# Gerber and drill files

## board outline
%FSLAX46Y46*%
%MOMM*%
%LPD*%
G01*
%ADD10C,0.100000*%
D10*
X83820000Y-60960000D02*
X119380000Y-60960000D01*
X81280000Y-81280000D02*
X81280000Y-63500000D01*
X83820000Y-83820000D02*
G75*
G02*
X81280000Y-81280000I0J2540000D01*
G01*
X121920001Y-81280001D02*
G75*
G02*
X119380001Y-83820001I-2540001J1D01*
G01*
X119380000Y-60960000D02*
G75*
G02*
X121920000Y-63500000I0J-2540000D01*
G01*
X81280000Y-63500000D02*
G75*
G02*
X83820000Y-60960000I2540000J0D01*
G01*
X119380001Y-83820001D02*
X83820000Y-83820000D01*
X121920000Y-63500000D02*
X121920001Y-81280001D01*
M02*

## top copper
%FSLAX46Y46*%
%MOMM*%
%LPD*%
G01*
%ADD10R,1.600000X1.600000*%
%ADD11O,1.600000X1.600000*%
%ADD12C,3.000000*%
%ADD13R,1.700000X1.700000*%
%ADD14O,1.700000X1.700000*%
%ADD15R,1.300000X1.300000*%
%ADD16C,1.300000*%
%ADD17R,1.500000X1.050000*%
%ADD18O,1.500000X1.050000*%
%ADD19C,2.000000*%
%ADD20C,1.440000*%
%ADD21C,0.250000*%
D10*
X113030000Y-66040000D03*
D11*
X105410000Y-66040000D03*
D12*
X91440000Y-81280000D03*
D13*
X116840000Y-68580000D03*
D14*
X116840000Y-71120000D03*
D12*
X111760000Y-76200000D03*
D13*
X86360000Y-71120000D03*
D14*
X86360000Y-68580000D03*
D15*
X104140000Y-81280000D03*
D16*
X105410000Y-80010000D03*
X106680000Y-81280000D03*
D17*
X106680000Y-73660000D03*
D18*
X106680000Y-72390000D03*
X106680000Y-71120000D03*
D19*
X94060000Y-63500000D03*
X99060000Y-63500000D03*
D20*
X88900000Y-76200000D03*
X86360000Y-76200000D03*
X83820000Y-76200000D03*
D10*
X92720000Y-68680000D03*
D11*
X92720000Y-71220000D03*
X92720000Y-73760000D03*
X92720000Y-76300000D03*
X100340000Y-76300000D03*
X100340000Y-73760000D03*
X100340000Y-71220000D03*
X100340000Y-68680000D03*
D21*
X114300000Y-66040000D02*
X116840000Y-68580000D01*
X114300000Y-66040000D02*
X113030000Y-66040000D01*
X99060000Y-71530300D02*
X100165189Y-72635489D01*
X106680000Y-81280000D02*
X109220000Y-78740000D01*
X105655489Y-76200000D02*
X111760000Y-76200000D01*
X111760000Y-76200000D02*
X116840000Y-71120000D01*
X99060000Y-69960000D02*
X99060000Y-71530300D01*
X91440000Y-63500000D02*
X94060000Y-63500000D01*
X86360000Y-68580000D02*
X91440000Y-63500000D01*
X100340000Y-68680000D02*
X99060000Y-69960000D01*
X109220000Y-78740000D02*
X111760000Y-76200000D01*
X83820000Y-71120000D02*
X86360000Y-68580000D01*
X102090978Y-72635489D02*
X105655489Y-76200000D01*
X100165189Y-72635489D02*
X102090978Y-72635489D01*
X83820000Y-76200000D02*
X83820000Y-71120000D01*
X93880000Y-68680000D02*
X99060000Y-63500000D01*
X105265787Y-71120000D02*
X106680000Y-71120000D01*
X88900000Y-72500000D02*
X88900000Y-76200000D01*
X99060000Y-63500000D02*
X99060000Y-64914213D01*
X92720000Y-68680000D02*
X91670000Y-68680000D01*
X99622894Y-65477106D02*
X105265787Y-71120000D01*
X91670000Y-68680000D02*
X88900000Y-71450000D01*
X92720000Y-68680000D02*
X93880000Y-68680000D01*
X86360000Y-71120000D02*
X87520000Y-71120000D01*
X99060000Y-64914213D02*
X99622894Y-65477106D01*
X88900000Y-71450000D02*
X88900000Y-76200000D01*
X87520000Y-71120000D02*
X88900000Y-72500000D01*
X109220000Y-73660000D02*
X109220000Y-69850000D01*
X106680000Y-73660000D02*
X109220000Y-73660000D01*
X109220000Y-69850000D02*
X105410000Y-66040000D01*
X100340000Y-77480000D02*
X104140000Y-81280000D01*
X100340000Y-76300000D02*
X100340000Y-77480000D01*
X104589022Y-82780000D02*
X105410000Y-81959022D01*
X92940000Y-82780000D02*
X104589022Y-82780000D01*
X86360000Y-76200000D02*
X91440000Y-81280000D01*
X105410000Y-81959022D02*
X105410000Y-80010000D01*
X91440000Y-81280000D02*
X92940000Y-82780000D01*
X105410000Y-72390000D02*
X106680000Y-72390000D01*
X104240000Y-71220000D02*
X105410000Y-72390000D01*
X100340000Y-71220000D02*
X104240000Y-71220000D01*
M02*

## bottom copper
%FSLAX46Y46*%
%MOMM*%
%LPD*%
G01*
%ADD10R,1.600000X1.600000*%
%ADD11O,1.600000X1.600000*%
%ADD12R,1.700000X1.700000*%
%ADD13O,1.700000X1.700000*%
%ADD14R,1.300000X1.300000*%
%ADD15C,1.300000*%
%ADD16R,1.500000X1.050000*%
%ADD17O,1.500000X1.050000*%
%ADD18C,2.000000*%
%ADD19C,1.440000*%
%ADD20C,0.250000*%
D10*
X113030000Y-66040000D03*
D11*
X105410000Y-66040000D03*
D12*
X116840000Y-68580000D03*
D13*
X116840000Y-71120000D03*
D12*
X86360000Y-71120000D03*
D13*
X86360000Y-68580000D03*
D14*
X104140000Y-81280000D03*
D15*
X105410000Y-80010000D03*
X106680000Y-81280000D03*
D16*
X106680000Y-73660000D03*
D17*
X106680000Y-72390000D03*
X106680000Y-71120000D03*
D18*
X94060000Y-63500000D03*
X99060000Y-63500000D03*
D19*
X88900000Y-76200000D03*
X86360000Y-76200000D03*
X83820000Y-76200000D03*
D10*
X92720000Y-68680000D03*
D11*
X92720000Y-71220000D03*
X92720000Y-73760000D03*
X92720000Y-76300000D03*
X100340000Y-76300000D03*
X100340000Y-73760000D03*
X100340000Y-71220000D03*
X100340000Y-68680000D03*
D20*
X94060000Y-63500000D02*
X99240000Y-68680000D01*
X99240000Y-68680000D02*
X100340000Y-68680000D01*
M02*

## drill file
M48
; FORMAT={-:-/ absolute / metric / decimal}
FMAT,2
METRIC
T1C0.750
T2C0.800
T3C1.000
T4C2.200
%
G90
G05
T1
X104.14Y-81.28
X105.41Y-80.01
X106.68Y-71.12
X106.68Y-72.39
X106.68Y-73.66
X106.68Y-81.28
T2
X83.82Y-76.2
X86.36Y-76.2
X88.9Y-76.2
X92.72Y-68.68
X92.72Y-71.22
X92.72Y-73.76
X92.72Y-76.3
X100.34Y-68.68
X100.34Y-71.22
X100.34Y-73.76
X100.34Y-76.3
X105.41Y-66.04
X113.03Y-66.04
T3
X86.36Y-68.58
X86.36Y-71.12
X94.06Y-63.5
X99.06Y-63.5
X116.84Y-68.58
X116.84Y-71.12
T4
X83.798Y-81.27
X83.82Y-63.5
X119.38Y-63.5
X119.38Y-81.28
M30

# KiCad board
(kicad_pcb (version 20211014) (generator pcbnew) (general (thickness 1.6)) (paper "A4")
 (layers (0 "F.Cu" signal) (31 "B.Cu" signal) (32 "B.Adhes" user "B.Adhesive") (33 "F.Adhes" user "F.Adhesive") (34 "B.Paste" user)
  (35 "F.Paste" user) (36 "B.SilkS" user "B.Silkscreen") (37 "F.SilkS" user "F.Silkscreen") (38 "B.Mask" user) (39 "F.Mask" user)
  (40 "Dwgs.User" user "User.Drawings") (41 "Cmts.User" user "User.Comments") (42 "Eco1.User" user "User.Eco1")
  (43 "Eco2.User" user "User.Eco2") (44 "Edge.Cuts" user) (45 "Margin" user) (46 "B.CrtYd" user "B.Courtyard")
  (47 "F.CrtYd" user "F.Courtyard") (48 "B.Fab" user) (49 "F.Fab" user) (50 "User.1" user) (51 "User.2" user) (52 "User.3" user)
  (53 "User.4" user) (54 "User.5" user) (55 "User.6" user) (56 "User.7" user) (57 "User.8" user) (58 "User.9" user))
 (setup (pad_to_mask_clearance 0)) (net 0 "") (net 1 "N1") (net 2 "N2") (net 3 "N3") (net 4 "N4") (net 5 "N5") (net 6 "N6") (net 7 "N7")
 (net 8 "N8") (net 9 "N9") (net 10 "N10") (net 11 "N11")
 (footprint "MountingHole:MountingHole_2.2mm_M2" (layer "F.Cu") (at 83.82 63.5)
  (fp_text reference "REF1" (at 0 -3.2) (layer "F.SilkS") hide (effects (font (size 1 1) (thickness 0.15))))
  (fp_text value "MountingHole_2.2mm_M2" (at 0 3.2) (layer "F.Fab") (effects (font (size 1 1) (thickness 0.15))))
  (pad "" np_thru_hole circle (at 0 0) (size 2.2 2.2) (drill 2.2) (layers *.Cu *.Mask)))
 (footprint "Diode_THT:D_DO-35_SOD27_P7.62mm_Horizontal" (layer "F.Cu") (at 113.03 66.04 180)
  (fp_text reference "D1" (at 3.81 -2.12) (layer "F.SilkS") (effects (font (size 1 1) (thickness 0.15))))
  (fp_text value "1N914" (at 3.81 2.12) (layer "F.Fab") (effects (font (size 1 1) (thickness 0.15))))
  (pad "1" thru_hole rect (at 0 0 180) (size 1.6 1.6) (drill 0.8) (layers *.Cu *.Mask) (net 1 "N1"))
  (pad "2" thru_hole oval (at 7.62 0 180) (size 1.6 1.6) (drill 0.8) (layers *.Cu *.Mask) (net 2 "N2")))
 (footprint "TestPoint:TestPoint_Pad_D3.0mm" (layer "F.Cu") (at 91.44 81.28)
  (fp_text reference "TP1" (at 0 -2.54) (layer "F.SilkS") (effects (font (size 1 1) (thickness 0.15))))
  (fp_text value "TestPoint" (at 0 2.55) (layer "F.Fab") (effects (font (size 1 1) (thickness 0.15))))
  (pad "1" smd circle (at 0 0) (size 3 3) (layers "F.Cu" "F.Mask") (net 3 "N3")))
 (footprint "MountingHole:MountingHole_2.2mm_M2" (layer "F.Cu") (at 119.38 63.5)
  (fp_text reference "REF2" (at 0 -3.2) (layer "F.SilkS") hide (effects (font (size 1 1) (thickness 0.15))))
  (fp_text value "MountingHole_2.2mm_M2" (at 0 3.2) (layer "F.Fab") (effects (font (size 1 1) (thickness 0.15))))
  (pad "" np_thru_hole circle (at 0 0) (size 2.2 2.2) (drill 2.2) (layers *.Cu *.Mask)))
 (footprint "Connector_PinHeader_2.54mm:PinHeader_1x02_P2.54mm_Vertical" (layer "F.Cu") (at 116.84 68.58)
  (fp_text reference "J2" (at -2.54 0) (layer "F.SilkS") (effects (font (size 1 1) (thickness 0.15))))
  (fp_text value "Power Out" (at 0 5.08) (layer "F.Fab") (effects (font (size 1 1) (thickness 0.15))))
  (pad "1" thru_hole rect (at 0 0) (size 1.7 1.7) (drill 1) (layers *.Cu *.Mask) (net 1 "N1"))
  (pad "2" thru_hole oval (at 0 2.54) (size 1.7 1.7) (drill 1) (layers *.Cu *.Mask) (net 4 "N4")))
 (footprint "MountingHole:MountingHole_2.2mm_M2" (layer "F.Cu") (at 119.38 81.28)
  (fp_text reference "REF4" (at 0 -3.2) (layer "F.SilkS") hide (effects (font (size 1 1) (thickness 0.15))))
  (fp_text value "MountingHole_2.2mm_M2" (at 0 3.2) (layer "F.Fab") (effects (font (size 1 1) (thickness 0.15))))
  (pad "" np_thru_hole circle (at 0 0) (size 2.2 2.2) (drill 2.2) (layers *.Cu *.Mask)))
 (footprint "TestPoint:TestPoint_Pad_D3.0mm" (layer "F.Cu") (at 111.76 76.2)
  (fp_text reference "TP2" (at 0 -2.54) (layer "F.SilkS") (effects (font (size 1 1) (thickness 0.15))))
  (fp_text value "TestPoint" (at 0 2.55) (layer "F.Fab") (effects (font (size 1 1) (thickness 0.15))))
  (pad "1" smd circle (at 0 0) (size 3 3) (layers "F.Cu" "F.Mask") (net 4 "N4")))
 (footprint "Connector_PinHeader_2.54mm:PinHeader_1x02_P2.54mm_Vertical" (layer "F.Cu") (at 86.36 71.12 180)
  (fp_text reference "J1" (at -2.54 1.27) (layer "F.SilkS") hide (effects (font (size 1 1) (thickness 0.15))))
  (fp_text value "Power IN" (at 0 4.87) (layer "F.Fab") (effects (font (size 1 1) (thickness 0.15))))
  (pad "1" thru_hole rect (at 0 0 180) (size 1.7 1.7) (drill 1) (layers *.Cu *.Mask) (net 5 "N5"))
  (pad "2" thru_hole oval (at 0 2.54 180) (size 1.7 1.7) (drill 1) (layers *.Cu *.Mask) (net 4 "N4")))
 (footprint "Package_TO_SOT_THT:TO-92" (layer "F.Cu") (at 104.14 81.28)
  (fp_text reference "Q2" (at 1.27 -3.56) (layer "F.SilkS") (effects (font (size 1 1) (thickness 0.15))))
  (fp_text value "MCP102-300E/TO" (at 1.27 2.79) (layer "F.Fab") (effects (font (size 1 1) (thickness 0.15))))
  (pad "1" thru_hole rect (at 0 0) (size 1.3 1.3) (drill 0.75) (layers *.Cu *.Mask) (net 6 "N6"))
  (pad "2" thru_hole circle (at 1.27 -1.27) (size 1.3 1.3) (drill 0.75) (layers *.Cu *.Mask) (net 3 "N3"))
  (pad "3" thru_hole circle (at 2.54 0) (size 1.3 1.3) (drill 0.75) (layers *.Cu *.Mask) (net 4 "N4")))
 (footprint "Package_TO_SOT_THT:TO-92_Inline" (layer "F.Cu") (at 106.68 73.66 90)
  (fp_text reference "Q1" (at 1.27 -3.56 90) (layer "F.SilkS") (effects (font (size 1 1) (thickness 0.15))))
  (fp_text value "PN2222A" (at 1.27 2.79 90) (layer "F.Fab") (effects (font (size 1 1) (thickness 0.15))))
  (pad "1" thru_hole rect (at 0 0 90) (size 1.05 1.5) (drill 0.75) (layers *.Cu *.Mask) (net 2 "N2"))
  (pad "2" thru_hole oval (at 1.27 0 90) (size 1.05 1.5) (drill 0.75) (layers *.Cu *.Mask) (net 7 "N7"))
  (pad "3" thru_hole oval (at 2.54 0 90) (size 1.05 1.5) (drill 0.75) (layers *.Cu *.Mask) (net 5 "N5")))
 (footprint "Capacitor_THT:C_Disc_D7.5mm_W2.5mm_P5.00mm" (layer "F.Cu") (at 94.06 63.5)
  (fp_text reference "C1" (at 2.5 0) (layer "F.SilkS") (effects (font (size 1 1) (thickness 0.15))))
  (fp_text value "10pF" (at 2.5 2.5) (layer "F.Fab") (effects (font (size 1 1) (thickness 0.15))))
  (pad "1" thru_hole circle (at 0 0) (size 2 2) (drill 1) (layers *.Cu *.Mask) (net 4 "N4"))
  (pad "2" thru_hole circle (at 5 0) (size 2 2) (drill 1) (layers *.Cu *.Mask) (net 5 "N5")))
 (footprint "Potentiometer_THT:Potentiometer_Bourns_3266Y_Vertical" (layer "F.Cu") (at 88.9 76.2)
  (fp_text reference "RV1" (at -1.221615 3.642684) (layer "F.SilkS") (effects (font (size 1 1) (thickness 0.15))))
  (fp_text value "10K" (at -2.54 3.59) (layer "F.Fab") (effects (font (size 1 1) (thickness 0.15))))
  (pad "1" thru_hole circle (at 0 0) (size 1.44 1.44) (drill 0.8) (layers *.Cu *.Mask) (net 5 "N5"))
  (pad "2" thru_hole circle (at -2.54 0) (size 1.44 1.44) (drill 0.8) (layers *.Cu *.Mask) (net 3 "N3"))
  (pad "3" thru_hole circle (at -5.08 0) (size 1.44 1.44) (drill 0.8) (layers *.Cu *.Mask) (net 4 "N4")))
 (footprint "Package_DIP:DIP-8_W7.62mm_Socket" (layer "F.Cu") (at 92.72 68.68)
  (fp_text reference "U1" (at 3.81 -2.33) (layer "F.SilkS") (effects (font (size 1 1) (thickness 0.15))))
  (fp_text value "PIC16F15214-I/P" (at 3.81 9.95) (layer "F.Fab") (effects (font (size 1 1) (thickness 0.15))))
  (pad "1" thru_hole rect (at 0 0) (size 1.6 1.6) (drill 0.8) (layers *.Cu *.Mask) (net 5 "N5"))
  (pad "2" thru_hole oval (at 0 2.54) (size 1.6 1.6) (drill 0.8) (layers *.Cu *.Mask) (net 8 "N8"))
  (pad "3" thru_hole oval (at 0 5.08) (size 1.6 1.6) (drill 0.8) (layers *.Cu *.Mask) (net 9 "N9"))
  (pad "4" thru_hole oval (at 0 7.62) (size 1.6 1.6) (drill 0.8) (layers *.Cu *.Mask) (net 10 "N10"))
  (pad "5" thru_hole oval (at 7.62 7.62) (size 1.6 1.6) (drill 0.8) (layers *.Cu *.Mask) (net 6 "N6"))
  (pad "6" thru_hole oval (at 7.62 5.08) (size 1.6 1.6) (drill 0.8) (layers *.Cu *.Mask) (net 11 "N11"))
  (pad "7" thru_hole oval (at 7.62 2.54) (size 1.6 1.6) (drill 0.8) (layers *.Cu *.Mask) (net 7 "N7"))
  (pad "8" thru_hole oval (at 7.62 0) (size 1.6 1.6) (drill 0.8) (layers *.Cu *.Mask) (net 4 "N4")))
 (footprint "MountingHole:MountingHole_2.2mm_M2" (layer "F.Cu") (at 83.798246 81.269655)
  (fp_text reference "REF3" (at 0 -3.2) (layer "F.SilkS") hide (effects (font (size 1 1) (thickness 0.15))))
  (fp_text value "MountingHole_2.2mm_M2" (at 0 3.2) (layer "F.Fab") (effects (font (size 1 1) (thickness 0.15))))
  (pad "" np_thru_hole circle (at 0 0) (size 2.2 2.2) (drill 2.2) (layers *.Cu *.Mask)))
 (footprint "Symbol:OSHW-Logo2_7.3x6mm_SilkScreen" (layer "B.Cu") (at 111.76 71.12 180)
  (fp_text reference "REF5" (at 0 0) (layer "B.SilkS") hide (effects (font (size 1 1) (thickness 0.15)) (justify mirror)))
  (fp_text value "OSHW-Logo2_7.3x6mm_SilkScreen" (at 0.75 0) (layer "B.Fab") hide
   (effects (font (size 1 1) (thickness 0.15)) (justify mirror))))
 (gr_line (start 83.82 60.96) (end 119.38 60.96) (layer "Edge.Cuts") (width 0.1))
 (gr_line (start 81.28 81.28) (end 81.28 63.5) (layer "Edge.Cuts") (width 0.1))
 (gr_arc (start 83.82 83.82) (mid 82.023949 83.076051) (end 81.28 81.28) (layer "Edge.Cuts") (width 0.1))
 (gr_arc (start 121.920001 81.280001) (mid 121.176052 83.076052) (end 119.380001 83.820001) (layer "Edge.Cuts") (width 0.1))
 (gr_arc (start 119.38 60.96) (mid 121.176051 61.703949) (end 121.92 63.5) (layer "Edge.Cuts") (width 0.1))
 (gr_arc (start 81.28 63.5) (mid 82.023949 61.703949) (end 83.82 60.96) (layer "Edge.Cuts") (width 0.1))
 (gr_line (start 119.380001 83.820001) (end 83.82 83.82) (layer "Edge.Cuts") (width 0.1))
 (gr_line (start 121.92 63.5) (end 121.920001 81.280001) (layer "Edge.Cuts") (width 0.1))
 (segment (start 114.3 66.04) (end 116.84 68.58) (width 0.25) (layer "F.Cu") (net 1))
 (segment (start 114.3 66.04) (end 113.03 66.04) (width 0.25) (layer "F.Cu") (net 1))
 (segment (start 99.06 71.5303) (end 100.165189 72.635489) (width 0.25) (layer "F.Cu") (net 4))
 (segment (start 106.68 81.28) (end 109.22 78.74) (width 0.25) (layer "F.Cu") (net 4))
 (segment (start 105.655489 76.2) (end 111.76 76.2) (width 0.25) (layer "F.Cu") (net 4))
 (segment (start 111.76 76.2) (end 116.84 71.12) (width 0.25) (layer "F.Cu") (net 4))
 (segment (start 99.06 69.96) (end 99.06 71.5303) (width 0.25) (layer "F.Cu") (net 4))
 (segment (start 91.44 63.5) (end 94.06 63.5) (width 0.25) (layer "F.Cu") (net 4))
 (segment (start 86.36 68.58) (end 91.44 63.5) (width 0.25) (layer "F.Cu") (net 4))
 (segment (start 100.34 68.68) (end 99.06 69.96) (width 0.25) (layer "F.Cu") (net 4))
 (segment (start 109.22 78.74) (end 111.76 76.2) (width 0.25) (layer "F.Cu") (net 4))
 (segment (start 83.82 71.12) (end 86.36 68.58) (width 0.25) (layer "F.Cu") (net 4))
 (segment (start 102.090978 72.635489) (end 105.655489 76.2) (width 0.25) (layer "F.Cu") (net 4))
 (segment (start 100.165189 72.635489) (end 102.090978 72.635489) (width 0.25) (layer "F.Cu") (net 4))
 (segment (start 83.82 76.2) (end 83.82 71.12) (width 0.25) (layer "F.Cu") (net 4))
 (segment (start 94.06 63.5) (end 99.24 68.68) (width 0.25) (layer "B.Cu") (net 4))
 (segment (start 99.24 68.68) (end 100.34 68.68) (width 0.25) (layer "B.Cu") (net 4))
 (segment (start 93.88 68.68) (end 99.06 63.5) (width 0.25) (layer "F.Cu") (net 5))
 (segment (start 105.265787 71.12) (end 106.68 71.12) (width 0.25) (layer "F.Cu") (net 5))
 (segment (start 88.9 72.5) (end 88.9 76.2) (width 0.25) (layer "F.Cu") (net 5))
 (segment (start 99.06 63.5) (end 99.06 64.914213) (width 0.25) (layer "F.Cu") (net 5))
 (segment (start 92.72 68.68) (end 91.67 68.68) (width 0.25) (layer "F.Cu") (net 5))
 (segment (start 99.622894 65.477106) (end 105.265787 71.12) (width 0.25) (layer "F.Cu") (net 5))
 (segment (start 91.67 68.68) (end 88.9 71.45) (width 0.25) (layer "F.Cu") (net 5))
 (segment (start 92.72 68.68) (end 93.88 68.68) (width 0.25) (layer "F.Cu") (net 5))
 (segment (start 86.36 71.12) (end 87.52 71.12) (width 0.25) (layer "F.Cu") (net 5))
 (segment (start 99.06 64.914213) (end 99.622894 65.477106) (width 0.25) (layer "F.Cu") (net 5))
 (segment (start 88.9 71.45) (end 88.9 76.2) (width 0.25) (layer "F.Cu") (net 5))
 (segment (start 87.52 71.12) (end 88.9 72.5) (width 0.25) (layer "F.Cu") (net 5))
 (segment (start 109.22 73.66) (end 109.22 69.85) (width 0.25) (layer "F.Cu") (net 2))
 (segment (start 106.68 73.66) (end 109.22 73.66) (width 0.25) (layer "F.Cu") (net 2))
 (segment (start 109.22 69.85) (end 105.41 66.04) (width 0.25) (layer "F.Cu") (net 2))
 (segment (start 100.34 77.48) (end 104.14 81.28) (width 0.25) (layer "F.Cu") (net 6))
 (segment (start 100.34 76.3) (end 100.34 77.48) (width 0.25) (layer "F.Cu") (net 6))
 (segment (start 104.589022 82.78) (end 105.41 81.959022) (width 0.25) (layer "F.Cu") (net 3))
 (segment (start 92.94 82.78) (end 104.589022 82.78) (width 0.25) (layer "F.Cu") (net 3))
 (segment (start 86.36 76.2) (end 91.44 81.28) (width 0.25) (layer "F.Cu") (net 3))
 (segment (start 105.41 81.959022) (end 105.41 80.01) (width 0.25) (layer "F.Cu") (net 3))
 (segment (start 91.44 81.28) (end 92.94 82.78) (width 0.25) (layer "F.Cu") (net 3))
 (segment (start 105.41 72.39) (end 106.68 72.39) (width 0.25) (layer "F.Cu") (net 7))
 (segment (start 104.24 71.22) (end 105.41 72.39) (width 0.25) (layer "F.Cu") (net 7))
 (segment (start 100.34 71.22) (end 104.24 71.22) (width 0.25) (layer "F.Cu") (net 7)))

